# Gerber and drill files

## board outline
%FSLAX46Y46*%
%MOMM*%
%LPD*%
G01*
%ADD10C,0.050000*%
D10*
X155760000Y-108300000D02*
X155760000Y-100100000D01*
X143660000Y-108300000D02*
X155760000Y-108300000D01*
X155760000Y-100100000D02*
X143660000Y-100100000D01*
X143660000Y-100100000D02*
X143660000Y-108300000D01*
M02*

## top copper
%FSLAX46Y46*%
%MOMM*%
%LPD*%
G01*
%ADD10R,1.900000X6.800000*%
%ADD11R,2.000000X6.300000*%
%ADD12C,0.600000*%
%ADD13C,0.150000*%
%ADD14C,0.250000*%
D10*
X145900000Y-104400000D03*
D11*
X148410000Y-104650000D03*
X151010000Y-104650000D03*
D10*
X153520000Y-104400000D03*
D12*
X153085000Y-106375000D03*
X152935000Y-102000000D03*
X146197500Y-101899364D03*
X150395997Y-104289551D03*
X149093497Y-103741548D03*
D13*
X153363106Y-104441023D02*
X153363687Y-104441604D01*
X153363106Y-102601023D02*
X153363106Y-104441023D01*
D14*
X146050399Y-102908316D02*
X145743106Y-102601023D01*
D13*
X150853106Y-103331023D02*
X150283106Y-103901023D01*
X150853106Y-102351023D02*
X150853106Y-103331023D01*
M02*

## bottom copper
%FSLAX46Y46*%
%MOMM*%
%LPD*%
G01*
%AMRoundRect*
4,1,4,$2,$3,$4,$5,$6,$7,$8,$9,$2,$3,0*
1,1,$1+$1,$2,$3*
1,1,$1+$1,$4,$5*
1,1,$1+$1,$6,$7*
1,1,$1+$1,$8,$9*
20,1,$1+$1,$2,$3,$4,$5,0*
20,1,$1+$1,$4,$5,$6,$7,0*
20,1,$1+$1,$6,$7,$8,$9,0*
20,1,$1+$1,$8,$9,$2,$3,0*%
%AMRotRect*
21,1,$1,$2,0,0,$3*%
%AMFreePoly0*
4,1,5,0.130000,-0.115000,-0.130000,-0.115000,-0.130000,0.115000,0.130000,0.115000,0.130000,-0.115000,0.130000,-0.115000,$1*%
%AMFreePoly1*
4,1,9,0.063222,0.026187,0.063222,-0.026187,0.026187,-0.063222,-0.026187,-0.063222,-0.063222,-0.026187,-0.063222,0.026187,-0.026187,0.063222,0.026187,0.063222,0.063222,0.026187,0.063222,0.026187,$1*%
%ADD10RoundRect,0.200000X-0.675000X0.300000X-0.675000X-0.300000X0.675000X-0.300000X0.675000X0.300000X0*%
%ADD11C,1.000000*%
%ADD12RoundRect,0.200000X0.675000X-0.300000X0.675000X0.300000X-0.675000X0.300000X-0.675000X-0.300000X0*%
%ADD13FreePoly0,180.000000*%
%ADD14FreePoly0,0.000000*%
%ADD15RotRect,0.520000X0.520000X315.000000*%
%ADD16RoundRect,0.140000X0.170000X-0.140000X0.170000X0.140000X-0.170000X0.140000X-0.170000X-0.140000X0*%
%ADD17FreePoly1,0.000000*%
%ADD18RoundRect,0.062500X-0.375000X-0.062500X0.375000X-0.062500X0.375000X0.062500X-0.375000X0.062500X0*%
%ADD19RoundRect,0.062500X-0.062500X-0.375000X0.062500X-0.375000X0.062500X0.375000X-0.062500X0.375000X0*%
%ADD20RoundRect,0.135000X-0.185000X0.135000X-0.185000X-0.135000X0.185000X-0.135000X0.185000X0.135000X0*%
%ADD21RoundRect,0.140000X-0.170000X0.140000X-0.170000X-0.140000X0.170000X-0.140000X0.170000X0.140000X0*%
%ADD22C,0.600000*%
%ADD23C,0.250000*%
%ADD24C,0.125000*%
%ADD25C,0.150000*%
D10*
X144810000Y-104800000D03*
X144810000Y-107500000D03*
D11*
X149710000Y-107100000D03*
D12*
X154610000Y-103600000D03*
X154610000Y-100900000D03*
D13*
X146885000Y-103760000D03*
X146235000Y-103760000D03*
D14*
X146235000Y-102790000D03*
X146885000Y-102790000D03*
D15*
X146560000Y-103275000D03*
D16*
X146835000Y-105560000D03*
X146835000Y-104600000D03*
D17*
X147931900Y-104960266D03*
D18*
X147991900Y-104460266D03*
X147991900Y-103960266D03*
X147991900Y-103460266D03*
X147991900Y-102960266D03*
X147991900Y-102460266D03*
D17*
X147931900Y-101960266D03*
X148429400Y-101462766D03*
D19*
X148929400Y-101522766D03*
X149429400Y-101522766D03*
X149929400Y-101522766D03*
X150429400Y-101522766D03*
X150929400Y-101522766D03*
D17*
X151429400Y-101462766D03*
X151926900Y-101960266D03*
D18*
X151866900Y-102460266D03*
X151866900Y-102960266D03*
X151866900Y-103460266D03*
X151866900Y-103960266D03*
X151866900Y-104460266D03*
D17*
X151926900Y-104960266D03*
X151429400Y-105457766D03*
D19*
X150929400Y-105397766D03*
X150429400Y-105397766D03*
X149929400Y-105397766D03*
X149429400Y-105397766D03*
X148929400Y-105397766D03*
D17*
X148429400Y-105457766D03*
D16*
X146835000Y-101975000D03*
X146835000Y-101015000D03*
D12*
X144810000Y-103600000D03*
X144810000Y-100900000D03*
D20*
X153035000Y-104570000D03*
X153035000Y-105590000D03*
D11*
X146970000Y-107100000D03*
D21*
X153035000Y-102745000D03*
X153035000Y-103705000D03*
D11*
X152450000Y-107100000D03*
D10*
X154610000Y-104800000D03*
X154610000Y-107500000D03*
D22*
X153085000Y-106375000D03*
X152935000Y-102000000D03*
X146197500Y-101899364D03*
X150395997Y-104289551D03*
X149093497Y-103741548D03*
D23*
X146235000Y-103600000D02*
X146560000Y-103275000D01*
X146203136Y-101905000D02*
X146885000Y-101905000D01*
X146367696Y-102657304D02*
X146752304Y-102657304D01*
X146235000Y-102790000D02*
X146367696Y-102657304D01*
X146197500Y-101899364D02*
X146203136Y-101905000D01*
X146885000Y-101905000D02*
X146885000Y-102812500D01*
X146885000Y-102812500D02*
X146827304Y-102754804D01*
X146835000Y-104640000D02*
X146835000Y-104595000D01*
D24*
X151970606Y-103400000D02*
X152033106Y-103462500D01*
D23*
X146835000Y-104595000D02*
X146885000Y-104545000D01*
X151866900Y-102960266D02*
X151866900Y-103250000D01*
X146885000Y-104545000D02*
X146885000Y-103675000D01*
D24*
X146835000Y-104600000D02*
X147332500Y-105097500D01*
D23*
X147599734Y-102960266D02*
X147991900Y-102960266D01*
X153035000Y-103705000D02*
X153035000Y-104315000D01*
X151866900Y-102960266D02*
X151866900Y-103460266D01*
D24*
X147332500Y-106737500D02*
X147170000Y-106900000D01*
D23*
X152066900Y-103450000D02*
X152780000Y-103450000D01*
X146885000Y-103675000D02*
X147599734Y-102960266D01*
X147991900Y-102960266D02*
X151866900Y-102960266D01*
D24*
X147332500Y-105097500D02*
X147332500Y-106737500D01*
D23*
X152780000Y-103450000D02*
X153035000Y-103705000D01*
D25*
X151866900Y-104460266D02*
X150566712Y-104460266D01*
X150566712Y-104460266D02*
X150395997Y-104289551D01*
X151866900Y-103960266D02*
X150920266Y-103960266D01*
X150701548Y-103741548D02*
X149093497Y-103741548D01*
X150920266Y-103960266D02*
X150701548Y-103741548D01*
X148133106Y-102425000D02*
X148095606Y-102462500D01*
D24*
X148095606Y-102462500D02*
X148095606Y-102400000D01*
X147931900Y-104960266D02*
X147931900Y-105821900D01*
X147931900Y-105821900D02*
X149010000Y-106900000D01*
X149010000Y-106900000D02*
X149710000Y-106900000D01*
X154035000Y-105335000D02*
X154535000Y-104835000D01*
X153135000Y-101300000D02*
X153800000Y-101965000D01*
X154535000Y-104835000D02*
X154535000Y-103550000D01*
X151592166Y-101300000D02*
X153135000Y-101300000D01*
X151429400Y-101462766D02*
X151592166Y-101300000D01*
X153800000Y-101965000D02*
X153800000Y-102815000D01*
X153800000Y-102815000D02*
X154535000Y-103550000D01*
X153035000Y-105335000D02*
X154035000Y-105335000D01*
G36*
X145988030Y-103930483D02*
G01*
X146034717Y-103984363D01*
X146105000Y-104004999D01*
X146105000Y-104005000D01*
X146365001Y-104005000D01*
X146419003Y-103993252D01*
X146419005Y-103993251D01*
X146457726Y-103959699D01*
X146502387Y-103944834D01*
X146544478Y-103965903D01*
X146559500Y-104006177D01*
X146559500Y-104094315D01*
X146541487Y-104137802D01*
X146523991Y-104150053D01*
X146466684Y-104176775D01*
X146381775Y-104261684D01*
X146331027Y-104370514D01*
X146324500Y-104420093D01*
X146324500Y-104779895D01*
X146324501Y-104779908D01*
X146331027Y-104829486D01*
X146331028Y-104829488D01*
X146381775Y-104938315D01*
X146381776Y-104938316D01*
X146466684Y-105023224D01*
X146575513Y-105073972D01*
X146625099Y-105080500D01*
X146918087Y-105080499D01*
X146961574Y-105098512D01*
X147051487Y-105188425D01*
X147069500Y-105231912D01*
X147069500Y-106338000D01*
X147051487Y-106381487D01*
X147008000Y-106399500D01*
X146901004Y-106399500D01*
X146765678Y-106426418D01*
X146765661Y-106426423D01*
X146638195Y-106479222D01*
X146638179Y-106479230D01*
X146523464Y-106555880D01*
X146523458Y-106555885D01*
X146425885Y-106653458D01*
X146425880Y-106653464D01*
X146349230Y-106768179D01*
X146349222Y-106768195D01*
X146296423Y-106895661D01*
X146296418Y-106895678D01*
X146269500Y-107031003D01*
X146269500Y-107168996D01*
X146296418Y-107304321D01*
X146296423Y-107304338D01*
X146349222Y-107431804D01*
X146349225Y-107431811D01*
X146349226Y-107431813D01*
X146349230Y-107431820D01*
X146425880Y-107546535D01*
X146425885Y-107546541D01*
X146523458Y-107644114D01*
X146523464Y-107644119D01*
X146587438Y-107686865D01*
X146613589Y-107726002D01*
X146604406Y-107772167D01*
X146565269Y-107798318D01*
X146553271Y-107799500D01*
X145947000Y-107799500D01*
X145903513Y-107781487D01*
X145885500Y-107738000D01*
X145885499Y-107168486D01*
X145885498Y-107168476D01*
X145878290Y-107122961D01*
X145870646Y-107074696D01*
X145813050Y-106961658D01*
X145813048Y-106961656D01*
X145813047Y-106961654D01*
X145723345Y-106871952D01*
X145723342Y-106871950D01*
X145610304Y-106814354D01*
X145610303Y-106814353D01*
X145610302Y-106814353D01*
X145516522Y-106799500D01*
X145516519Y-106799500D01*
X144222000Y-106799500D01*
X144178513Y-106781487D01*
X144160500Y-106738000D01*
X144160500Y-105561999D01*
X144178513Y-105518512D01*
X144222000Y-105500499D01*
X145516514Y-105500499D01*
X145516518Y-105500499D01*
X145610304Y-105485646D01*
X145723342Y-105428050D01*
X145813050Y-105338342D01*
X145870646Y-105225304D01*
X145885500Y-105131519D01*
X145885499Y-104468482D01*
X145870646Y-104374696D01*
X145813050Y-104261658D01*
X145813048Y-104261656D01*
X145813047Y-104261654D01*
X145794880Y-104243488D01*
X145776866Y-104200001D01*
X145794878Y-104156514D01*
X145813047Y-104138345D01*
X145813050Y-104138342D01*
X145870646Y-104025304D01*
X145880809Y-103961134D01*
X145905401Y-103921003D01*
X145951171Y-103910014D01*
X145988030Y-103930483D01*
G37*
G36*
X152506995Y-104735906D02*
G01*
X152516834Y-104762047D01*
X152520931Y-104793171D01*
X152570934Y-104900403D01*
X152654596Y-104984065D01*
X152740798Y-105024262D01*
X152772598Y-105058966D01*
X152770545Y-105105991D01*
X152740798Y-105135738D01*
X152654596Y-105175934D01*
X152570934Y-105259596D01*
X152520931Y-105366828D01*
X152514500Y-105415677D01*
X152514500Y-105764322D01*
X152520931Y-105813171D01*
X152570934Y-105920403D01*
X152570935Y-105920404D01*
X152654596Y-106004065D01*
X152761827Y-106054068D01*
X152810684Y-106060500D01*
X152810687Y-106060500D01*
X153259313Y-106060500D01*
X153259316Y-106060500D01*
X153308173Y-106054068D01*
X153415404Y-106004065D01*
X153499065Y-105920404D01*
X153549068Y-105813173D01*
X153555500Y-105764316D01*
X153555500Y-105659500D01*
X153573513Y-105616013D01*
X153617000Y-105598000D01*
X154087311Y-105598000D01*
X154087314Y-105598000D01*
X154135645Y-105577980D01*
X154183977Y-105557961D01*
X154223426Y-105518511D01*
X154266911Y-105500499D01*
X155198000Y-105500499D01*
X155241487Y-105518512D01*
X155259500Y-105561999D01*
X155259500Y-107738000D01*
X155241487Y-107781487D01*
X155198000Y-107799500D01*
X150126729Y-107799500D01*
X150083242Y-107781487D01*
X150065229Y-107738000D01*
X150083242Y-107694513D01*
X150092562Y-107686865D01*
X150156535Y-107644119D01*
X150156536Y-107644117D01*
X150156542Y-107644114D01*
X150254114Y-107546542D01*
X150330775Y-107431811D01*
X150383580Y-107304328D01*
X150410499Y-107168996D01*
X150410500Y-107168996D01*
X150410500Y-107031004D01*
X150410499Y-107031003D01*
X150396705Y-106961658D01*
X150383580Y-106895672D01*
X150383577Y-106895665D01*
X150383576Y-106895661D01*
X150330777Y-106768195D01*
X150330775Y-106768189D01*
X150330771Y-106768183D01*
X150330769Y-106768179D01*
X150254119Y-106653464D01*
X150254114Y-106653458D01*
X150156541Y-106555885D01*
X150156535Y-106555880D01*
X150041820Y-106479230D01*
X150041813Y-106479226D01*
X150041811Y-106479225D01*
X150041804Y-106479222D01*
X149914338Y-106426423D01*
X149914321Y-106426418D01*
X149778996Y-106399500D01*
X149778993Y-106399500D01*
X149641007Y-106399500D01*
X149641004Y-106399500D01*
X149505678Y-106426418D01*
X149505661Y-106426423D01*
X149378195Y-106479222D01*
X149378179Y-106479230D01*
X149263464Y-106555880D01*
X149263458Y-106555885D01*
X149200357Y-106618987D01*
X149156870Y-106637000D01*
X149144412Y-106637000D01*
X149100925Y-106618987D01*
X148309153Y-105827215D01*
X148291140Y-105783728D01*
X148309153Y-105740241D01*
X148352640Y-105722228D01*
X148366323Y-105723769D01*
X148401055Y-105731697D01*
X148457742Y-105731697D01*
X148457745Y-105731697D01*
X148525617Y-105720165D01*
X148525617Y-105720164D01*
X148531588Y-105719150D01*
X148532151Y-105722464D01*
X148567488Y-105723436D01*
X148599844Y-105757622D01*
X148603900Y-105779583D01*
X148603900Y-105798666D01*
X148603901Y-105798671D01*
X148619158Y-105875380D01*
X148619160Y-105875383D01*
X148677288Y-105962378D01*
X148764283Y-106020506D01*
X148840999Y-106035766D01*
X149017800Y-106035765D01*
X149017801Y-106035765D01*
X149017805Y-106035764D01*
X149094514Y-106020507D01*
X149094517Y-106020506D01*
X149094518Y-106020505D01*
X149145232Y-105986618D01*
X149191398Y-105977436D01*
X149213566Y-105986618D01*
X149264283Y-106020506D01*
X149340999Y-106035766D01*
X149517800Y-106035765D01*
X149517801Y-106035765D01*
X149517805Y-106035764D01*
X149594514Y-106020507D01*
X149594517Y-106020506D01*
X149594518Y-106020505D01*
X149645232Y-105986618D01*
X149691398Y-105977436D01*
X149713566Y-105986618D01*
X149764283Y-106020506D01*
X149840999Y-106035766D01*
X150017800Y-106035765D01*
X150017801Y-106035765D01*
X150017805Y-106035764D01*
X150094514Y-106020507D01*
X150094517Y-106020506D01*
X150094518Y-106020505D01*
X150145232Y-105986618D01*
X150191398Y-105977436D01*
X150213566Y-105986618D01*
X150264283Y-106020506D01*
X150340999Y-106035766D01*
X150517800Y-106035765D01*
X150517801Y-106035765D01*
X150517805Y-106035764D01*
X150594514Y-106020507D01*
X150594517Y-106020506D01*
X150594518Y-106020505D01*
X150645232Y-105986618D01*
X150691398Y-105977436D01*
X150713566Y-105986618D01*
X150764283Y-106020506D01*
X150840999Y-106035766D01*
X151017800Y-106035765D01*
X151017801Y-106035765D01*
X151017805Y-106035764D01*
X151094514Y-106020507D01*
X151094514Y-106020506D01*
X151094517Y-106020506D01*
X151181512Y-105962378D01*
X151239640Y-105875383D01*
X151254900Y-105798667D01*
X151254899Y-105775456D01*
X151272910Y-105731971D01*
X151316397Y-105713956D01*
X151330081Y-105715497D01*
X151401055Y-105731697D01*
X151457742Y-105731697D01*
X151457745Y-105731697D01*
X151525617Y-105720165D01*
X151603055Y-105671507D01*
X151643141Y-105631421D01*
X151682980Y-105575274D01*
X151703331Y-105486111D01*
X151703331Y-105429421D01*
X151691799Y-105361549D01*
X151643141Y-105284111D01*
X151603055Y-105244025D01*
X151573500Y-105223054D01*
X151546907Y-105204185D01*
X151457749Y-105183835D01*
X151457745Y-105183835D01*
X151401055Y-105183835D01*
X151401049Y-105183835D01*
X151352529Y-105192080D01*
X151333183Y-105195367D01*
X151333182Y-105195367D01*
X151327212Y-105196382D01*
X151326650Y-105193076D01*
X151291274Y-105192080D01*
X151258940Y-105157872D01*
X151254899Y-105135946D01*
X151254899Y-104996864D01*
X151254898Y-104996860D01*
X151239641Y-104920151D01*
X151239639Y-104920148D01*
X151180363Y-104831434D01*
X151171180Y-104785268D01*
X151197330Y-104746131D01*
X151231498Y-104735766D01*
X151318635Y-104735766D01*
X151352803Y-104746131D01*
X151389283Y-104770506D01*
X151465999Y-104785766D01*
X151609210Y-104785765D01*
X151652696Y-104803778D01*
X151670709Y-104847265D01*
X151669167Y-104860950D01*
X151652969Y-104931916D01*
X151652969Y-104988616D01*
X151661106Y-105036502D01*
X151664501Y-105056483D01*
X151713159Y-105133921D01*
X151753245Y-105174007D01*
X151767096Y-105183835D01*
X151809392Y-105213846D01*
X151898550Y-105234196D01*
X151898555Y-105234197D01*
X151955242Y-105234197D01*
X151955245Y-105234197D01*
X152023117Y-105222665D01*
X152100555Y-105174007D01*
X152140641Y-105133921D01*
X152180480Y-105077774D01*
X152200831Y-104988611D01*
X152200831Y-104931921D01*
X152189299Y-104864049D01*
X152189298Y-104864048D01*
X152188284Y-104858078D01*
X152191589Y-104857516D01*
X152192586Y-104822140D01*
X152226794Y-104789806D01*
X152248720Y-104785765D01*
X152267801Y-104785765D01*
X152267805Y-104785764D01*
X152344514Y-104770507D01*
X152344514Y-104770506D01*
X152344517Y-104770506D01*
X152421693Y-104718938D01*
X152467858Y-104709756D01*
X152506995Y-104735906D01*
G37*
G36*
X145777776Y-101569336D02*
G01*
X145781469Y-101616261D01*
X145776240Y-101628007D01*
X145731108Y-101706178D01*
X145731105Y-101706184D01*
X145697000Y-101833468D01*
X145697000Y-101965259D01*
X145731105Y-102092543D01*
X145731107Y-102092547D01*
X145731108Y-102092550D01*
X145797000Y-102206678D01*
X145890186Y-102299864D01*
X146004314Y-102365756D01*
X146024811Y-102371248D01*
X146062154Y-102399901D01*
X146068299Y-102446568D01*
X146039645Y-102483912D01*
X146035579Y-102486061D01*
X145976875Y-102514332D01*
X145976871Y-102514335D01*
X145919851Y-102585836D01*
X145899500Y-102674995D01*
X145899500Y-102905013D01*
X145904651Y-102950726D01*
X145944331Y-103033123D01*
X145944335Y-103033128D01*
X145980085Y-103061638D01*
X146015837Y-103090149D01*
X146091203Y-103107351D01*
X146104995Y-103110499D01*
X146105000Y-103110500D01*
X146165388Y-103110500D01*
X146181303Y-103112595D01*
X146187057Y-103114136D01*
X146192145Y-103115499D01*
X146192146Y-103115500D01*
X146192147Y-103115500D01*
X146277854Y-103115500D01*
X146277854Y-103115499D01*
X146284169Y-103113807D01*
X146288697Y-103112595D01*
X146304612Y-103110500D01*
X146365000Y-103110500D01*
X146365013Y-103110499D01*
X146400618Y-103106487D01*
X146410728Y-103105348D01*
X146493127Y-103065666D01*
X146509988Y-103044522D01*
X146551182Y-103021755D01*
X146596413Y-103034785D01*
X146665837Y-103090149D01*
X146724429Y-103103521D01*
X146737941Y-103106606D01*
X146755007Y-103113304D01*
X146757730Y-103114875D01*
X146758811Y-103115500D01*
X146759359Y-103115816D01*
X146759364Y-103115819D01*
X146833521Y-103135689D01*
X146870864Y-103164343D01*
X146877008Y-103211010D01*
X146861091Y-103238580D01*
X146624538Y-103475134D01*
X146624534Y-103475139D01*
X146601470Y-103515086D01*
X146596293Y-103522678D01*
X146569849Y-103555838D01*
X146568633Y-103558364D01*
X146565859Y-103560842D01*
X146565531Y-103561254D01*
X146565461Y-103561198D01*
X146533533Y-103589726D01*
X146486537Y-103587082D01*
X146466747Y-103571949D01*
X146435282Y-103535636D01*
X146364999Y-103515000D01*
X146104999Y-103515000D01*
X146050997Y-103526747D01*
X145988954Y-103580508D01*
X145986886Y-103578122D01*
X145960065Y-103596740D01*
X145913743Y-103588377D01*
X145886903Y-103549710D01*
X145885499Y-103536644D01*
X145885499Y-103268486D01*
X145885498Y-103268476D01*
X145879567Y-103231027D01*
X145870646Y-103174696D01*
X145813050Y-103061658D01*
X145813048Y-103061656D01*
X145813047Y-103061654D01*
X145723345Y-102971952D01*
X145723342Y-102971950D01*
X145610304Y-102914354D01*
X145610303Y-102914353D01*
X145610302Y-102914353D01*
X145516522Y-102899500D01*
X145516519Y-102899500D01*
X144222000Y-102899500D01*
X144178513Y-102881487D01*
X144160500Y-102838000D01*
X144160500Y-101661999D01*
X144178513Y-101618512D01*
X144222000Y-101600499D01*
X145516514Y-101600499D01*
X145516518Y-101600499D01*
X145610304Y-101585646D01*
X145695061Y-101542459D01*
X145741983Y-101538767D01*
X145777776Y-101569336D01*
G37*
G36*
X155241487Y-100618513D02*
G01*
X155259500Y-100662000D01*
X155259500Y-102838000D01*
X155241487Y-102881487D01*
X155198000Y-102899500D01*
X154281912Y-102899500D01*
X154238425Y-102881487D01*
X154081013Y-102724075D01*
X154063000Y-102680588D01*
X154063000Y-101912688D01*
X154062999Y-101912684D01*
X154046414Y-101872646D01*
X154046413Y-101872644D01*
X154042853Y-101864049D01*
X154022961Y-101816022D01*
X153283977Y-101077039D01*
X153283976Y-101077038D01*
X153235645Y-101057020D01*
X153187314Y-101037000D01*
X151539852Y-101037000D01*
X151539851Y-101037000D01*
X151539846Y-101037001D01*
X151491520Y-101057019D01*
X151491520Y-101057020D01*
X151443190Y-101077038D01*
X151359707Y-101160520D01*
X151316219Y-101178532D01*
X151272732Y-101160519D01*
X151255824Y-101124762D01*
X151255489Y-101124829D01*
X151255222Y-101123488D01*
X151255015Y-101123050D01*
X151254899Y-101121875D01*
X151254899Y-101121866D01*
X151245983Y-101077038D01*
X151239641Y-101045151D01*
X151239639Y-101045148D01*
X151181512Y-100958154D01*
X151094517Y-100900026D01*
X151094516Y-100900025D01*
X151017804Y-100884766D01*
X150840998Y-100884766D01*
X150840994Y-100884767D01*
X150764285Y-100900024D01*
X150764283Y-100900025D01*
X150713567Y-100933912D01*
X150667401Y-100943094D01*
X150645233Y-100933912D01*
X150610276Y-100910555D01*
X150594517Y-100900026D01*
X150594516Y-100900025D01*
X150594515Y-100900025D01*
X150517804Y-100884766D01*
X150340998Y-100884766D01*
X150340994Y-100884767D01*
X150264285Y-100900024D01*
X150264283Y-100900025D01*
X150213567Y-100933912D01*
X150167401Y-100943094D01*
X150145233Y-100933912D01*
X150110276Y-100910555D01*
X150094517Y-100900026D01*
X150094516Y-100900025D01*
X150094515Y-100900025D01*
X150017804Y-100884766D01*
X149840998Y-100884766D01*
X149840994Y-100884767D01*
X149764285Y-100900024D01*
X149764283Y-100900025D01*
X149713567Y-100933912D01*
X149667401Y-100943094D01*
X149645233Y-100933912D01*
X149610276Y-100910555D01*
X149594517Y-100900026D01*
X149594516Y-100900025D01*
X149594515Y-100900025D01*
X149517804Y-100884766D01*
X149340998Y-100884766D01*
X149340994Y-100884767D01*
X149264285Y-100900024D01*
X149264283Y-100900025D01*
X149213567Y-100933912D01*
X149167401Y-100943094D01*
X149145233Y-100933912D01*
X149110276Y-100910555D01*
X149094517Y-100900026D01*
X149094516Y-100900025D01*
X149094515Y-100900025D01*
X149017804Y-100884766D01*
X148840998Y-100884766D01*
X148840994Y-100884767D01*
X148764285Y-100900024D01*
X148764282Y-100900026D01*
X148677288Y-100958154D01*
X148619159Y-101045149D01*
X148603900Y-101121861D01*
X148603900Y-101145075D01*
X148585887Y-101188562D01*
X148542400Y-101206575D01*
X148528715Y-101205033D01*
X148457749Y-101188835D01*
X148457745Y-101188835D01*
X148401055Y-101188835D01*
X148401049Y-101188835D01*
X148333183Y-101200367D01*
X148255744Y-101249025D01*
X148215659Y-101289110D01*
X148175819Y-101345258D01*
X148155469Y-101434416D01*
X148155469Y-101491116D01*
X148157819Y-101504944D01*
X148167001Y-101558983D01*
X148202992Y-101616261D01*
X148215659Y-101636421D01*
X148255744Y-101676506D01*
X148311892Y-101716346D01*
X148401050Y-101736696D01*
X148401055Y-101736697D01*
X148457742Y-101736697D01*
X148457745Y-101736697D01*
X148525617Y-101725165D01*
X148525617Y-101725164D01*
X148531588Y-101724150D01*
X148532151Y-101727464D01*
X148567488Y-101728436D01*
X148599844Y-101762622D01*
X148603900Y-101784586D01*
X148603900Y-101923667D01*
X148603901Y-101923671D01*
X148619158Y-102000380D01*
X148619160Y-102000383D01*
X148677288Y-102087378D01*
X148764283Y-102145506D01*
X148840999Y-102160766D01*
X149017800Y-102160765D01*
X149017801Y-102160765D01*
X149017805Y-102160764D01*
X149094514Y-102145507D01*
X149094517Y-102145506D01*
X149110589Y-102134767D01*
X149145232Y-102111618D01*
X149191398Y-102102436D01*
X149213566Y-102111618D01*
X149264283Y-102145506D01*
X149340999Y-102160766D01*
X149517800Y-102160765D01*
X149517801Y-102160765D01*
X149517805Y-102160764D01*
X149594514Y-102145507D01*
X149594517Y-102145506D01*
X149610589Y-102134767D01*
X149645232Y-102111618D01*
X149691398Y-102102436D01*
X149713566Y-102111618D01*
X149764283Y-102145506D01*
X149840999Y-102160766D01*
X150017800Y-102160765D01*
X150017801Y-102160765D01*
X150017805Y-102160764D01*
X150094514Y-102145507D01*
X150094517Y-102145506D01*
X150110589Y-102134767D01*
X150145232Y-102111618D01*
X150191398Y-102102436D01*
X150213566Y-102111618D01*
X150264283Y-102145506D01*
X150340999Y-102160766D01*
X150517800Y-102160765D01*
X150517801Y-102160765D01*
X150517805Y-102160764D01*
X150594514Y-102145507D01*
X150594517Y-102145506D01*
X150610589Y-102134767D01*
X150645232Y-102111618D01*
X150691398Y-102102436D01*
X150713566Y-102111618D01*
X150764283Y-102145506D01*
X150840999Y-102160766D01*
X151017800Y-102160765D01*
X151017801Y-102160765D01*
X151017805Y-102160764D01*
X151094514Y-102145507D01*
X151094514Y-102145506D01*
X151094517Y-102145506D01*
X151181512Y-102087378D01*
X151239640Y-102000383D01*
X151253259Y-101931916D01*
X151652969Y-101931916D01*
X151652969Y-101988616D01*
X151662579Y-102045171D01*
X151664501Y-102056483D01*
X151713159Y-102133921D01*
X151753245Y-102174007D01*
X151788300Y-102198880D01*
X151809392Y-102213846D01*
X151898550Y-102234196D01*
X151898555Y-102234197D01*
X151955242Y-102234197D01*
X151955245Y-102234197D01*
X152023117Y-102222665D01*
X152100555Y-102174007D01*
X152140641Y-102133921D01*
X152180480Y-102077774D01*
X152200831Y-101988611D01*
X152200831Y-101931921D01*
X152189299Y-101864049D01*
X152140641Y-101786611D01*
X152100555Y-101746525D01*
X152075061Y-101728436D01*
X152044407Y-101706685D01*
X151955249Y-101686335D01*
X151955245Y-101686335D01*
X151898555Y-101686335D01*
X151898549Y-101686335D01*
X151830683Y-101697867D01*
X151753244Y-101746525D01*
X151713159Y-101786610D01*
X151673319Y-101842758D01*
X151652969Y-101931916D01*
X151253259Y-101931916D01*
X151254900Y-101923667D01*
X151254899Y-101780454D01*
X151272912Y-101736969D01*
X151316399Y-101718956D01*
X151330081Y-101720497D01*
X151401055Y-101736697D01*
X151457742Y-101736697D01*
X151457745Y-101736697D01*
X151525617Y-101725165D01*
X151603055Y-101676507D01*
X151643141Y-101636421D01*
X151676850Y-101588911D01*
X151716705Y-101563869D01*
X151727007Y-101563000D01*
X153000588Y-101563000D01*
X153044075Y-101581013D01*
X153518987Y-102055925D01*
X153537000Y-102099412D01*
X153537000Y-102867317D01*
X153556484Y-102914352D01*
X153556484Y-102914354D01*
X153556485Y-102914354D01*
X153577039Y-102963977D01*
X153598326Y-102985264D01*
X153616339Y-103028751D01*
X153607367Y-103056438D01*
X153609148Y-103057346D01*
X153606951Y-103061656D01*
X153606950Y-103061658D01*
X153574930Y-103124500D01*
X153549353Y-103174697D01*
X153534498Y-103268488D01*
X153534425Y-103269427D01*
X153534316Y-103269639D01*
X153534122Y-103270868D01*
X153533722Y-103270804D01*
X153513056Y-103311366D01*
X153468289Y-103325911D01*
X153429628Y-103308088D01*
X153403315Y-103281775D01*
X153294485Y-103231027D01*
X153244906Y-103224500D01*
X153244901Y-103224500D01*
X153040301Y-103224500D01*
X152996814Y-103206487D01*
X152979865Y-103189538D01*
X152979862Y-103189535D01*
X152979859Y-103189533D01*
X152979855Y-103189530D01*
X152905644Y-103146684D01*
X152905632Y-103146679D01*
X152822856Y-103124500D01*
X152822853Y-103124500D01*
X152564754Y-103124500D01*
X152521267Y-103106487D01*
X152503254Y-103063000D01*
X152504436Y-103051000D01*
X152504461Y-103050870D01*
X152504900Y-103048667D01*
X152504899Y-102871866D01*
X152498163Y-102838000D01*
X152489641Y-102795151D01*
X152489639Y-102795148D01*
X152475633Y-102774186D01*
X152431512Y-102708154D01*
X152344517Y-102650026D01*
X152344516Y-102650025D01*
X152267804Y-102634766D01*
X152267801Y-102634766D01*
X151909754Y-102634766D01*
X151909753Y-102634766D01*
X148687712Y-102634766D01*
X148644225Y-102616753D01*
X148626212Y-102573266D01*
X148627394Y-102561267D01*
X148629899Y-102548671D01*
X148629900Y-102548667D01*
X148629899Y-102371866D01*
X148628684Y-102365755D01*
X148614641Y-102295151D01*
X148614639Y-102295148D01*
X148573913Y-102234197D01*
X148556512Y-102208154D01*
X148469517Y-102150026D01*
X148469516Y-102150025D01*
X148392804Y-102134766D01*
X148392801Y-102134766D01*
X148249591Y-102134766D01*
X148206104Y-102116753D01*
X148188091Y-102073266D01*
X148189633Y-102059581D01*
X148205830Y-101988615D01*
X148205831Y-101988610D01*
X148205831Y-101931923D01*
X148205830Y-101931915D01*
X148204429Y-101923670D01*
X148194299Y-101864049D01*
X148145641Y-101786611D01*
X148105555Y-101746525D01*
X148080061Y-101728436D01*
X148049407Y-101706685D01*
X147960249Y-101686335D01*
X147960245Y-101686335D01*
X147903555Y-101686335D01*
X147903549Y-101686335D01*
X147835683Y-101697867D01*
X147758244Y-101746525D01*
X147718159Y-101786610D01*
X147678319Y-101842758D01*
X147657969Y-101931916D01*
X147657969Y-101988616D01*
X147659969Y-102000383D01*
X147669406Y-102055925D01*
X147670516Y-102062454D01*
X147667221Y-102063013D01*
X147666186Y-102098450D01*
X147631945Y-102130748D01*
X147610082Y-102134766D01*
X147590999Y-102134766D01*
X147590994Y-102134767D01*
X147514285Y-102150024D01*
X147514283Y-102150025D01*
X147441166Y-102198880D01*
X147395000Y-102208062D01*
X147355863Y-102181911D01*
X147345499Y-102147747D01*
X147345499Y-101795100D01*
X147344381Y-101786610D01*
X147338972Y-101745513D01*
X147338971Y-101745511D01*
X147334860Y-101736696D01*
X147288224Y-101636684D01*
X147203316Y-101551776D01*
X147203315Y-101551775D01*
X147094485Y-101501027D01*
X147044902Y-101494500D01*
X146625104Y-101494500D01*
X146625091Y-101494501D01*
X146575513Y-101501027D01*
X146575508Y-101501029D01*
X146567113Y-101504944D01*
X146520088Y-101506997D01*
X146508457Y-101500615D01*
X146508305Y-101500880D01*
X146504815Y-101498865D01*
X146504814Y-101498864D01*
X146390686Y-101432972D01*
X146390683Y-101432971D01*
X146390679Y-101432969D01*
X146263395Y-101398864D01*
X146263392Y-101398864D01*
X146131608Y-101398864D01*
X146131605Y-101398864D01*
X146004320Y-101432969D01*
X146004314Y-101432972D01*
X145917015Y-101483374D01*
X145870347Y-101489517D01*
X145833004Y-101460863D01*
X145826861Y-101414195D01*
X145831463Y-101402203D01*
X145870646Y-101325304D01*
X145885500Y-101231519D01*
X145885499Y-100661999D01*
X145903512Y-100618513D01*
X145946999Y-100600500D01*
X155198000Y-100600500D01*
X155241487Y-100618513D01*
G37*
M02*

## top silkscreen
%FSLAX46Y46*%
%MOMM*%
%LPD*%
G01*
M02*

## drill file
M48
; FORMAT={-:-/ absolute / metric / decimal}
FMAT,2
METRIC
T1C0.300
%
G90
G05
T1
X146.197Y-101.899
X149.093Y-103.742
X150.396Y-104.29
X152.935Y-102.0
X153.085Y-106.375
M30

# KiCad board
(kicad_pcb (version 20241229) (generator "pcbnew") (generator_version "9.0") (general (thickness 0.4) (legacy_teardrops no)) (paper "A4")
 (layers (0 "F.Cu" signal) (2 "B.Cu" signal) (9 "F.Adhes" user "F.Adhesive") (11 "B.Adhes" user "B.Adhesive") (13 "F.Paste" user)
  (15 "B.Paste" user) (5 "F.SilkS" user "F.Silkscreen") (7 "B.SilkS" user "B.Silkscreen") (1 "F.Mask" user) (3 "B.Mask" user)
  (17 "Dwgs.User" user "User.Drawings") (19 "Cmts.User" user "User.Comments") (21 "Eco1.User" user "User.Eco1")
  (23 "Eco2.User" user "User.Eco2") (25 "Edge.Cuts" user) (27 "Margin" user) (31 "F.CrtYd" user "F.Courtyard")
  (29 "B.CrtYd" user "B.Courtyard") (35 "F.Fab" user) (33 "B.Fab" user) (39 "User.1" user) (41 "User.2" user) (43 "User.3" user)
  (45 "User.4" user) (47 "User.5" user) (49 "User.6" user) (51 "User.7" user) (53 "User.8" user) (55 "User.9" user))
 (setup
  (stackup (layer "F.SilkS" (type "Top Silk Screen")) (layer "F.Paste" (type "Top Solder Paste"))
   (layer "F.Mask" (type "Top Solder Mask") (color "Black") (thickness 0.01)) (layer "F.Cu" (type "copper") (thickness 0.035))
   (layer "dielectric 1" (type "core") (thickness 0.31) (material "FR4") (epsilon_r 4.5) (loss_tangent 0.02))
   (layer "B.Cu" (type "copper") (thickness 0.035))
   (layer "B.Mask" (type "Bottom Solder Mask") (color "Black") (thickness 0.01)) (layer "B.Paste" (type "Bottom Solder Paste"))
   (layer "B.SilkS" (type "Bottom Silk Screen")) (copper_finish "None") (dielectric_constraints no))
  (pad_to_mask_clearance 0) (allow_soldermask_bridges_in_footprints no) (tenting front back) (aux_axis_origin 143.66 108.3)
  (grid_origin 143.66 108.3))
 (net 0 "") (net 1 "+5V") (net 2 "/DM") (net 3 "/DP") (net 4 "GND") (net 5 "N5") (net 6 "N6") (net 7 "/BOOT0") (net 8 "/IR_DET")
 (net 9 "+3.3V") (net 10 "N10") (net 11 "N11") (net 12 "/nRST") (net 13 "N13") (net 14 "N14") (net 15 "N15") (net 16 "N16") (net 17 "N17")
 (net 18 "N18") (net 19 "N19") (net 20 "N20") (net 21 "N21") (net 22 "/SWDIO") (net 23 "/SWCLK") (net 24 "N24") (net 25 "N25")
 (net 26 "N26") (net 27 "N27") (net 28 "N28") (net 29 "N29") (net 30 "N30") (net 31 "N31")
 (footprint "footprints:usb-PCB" (layer "F.Cu") (at 149.71 100.1 180)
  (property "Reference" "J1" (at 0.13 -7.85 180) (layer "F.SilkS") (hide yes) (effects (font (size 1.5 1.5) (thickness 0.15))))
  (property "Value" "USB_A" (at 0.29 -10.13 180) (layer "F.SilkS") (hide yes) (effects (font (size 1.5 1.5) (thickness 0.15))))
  (pad "1" connect rect (at 3.81 -4.3 180) (size 1.9 6.8) (layers "F.Cu" "F.Mask") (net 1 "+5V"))
  (pad "2" connect rect (at 1.3 -4.55 180) (size 2 6.3) (layers "F.Cu" "F.Mask") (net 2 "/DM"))
  (pad "3" connect rect (at -1.3 -4.55 180) (size 2 6.3) (layers "F.Cu" "F.Mask") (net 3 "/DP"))
  (pad "4" connect rect (at -3.81 -4.3 180) (size 1.9 6.8) (layers "F.Cu" "F.Mask") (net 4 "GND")))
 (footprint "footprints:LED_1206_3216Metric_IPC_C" (layer "B.Cu") (at 144.81 106.15 -90)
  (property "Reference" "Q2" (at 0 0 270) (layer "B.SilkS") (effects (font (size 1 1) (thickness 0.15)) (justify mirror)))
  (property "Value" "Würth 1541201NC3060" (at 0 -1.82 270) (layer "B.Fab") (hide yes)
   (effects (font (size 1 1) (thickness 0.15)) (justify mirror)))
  (pad "1" smd roundrect (at -1.35 0 270) (size 1 1.75) (layers "B.Cu" "B.Mask" "B.Paste") (roundrect_rratio 0.2) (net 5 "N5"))
  (pad "2" smd roundrect (at 1.35 0 270) (size 1 1.75) (layers "B.Cu" "B.Mask" "B.Paste") (roundrect_rratio 0.2) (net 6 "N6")))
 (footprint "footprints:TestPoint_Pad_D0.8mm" (layer "B.Cu") (at 150.01 106.55 180)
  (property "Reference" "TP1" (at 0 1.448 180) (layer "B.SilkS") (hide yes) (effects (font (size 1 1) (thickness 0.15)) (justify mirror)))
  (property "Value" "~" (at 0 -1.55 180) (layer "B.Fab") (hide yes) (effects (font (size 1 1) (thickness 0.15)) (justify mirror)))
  (pad "1" smd circle (at 0.3 -0.55 180) (size 1 1) (layers "B.Cu" "B.Mask") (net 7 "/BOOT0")))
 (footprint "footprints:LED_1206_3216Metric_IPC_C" (layer "B.Cu") (at 154.61 102.25 90)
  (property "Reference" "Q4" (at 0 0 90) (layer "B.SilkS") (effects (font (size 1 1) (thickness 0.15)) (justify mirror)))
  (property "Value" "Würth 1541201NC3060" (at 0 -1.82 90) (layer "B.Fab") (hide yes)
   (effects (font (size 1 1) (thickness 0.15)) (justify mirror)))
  (pad "1" smd roundrect (at -1.35 0 90) (size 1 1.75) (layers "B.Cu" "B.Mask" "B.Paste") (roundrect_rratio 0.2) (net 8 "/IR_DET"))
  (pad "2" smd roundrect (at 1.35 0 90) (size 1 1.75) (layers "B.Cu" "B.Mask" "B.Paste") (roundrect_rratio 0.2) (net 4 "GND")))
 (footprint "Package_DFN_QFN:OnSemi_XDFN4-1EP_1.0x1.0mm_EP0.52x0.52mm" (layer "B.Cu") (at 146.56 103.275 90)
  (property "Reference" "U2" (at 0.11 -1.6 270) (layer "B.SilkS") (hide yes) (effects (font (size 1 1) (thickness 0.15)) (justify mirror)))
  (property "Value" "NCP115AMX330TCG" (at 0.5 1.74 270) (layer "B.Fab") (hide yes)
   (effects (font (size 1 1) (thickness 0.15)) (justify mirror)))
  (pad "1" smd custom (at -0.485 0.325 180) (size 0.26 0.23) (layers "B.Cu" "B.Mask" "B.Paste") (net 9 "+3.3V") (zone_connect 0)
   (thermal_bridge_angle 45) (options (clearance outline) (anchor rect)) (primitives))
  (pad "2" smd custom (at -0.485 -0.325 180) (size 0.26 0.23) (layers "B.Cu" "B.Mask" "B.Paste") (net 4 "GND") (zone_connect 0)
   (thermal_bridge_angle 45) (options (clearance outline) (anchor rect)) (primitives))
  (pad "3" smd custom (at 0.485 -0.325) (size 0.26 0.23) (layers "B.Cu" "B.Mask" "B.Paste") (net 1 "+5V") (zone_connect 0)
   (thermal_bridge_angle 45) (options (clearance outline) (anchor rect)) (primitives))
  (pad "4" smd custom (at 0.485 0.325) (size 0.26 0.23) (layers "B.Cu" "B.Mask" "B.Paste") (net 1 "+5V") (zone_connect 0)
   (thermal_bridge_angle 45) (options (clearance outline) (anchor rect)) (primitives))
  (pad "5" smd rect (at 0 0 315) (size 0.52 0.52) (layers "B.Cu" "B.Mask" "B.Paste") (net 4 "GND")))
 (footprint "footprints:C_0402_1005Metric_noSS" (layer "B.Cu") (at 146.835 105.08 90)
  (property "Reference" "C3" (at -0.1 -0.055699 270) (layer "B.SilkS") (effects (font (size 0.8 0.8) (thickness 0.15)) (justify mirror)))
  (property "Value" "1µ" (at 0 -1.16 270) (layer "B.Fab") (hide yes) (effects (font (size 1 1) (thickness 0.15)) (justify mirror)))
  (pad "1" smd roundrect (at -0.48 0 90) (size 0.56 0.62) (layers "B.Cu" "B.Mask" "B.Paste") (roundrect_rratio 0.25) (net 4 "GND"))
  (pad "2" smd roundrect (at 0.48 0 90) (size 0.56 0.62) (layers "B.Cu" "B.Mask" "B.Paste") (roundrect_rratio 0.25) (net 9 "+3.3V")))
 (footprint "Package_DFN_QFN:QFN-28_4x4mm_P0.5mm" (layer "B.Cu") (at 149.9294 103.460266)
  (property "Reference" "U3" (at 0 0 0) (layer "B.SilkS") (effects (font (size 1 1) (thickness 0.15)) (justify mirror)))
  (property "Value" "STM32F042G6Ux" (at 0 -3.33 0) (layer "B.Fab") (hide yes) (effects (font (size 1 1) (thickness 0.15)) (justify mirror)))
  (pad "1" smd custom (at -1.9975 1.5) (size 0.136863 0.136863) (layers "B.Cu" "B.Mask" "B.Paste") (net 7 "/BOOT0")
   (options (clearance outline) (anchor circle)) (primitives))
  (pad "2" smd roundrect (at -1.9375 1) (size 0.875 0.25) (layers "B.Cu" "B.Mask" "B.Paste") (roundrect_rratio 0.25) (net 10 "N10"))
  (pad "3" smd roundrect (at -1.9375 0.5) (size 0.875 0.25) (layers "B.Cu" "B.Mask" "B.Paste") (roundrect_rratio 0.25) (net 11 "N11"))
  (pad "4" smd roundrect (at -1.9375 0) (size 0.875 0.25) (layers "B.Cu" "B.Mask" "B.Paste") (roundrect_rratio 0.25) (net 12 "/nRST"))
  (pad "5" smd roundrect (at -1.9375 -0.5) (size 0.875 0.25) (layers "B.Cu" "B.Mask" "B.Paste") (roundrect_rratio 0.25) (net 9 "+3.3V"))
  (pad "6" smd roundrect (at -1.9375 -1) (size 0.875 0.25) (layers "B.Cu" "B.Mask" "B.Paste") (roundrect_rratio 0.25) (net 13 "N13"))
  (pad "7" smd custom (at -1.9975 -1.5) (size 0.136863 0.136863) (layers "B.Cu" "B.Mask" "B.Paste") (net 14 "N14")
   (options (clearance outline) (anchor circle)) (primitives))
  (pad "8" smd custom (at -1.5 -1.9975) (size 0.136863 0.136863) (layers "B.Cu" "B.Mask" "B.Paste") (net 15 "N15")
   (options (clearance outline) (anchor circle)) (primitives))
  (pad "9" smd roundrect (at -1 -1.9375) (size 0.25 0.875) (layers "B.Cu" "B.Mask" "B.Paste") (roundrect_rratio 0.25) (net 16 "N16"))
  (pad "10" smd roundrect (at -0.5 -1.9375) (size 0.25 0.875) (layers "B.Cu" "B.Mask" "B.Paste") (roundrect_rratio 0.25) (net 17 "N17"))
  (pad "11" smd roundrect (at 0 -1.9375) (size 0.25 0.875) (layers "B.Cu" "B.Mask" "B.Paste") (roundrect_rratio 0.25) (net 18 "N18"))
  (pad "12" smd roundrect (at 0.5 -1.9375) (size 0.25 0.875) (layers "B.Cu" "B.Mask" "B.Paste") (roundrect_rratio 0.25) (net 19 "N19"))
  (pad "13" smd roundrect (at 1 -1.9375) (size 0.25 0.875) (layers "B.Cu" "B.Mask" "B.Paste") (roundrect_rratio 0.25) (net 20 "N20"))
  (pad "14" smd custom (at 1.5 -1.9975) (size 0.136863 0.136863) (layers "B.Cu" "B.Mask" "B.Paste") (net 8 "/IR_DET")
   (options (clearance outline) (anchor circle)) (primitives))
  (pad "15" smd custom (at 1.9975 -1.5) (size 0.136863 0.136863) (layers "B.Cu" "B.Mask" "B.Paste") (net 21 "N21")
   (options (clearance outline) (anchor circle)) (primitives))
  (pad "16" smd roundrect (at 1.9375 -1) (size 0.875 0.25) (layers "B.Cu" "B.Mask" "B.Paste") (roundrect_rratio 0.25) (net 4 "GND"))
  (pad "17" smd roundrect (at 1.9375 -0.5) (size 0.875 0.25) (layers "B.Cu" "B.Mask" "B.Paste") (roundrect_rratio 0.25) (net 9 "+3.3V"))
  (pad "18" smd roundrect (at 1.9375 0) (size 0.875 0.25) (layers "B.Cu" "B.Mask" "B.Paste") (roundrect_rratio 0.25) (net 9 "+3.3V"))
  (pad "19" smd roundrect (at 1.9375 0.5) (size 0.875 0.25) (layers "B.Cu" "B.Mask" "B.Paste") (roundrect_rratio 0.25) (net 2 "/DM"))
  (pad "20" smd roundrect (at 1.9375 1) (size 0.875 0.25) (layers "B.Cu" "B.Mask" "B.Paste") (roundrect_rratio 0.25) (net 3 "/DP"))
  (pad "21" smd custom (at 1.9975 1.5) (size 0.136863 0.136863) (layers "B.Cu" "B.Mask" "B.Paste") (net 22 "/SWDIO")
   (options (clearance outline) (anchor circle)) (primitives))
  (pad "22" smd custom (at 1.5 1.9975) (size 0.136863 0.136863) (layers "B.Cu" "B.Mask" "B.Paste") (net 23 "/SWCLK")
   (options (clearance outline) (anchor circle)) (primitives))
  (pad "23" smd roundrect (at 1 1.9375) (size 0.25 0.875) (layers "B.Cu" "B.Mask" "B.Paste") (roundrect_rratio 0.25) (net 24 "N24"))
  (pad "24" smd roundrect (at 0.5 1.9375) (size 0.25 0.875) (layers "B.Cu" "B.Mask" "B.Paste") (roundrect_rratio 0.25) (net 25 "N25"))
  (pad "25" smd roundrect (at 0 1.9375) (size 0.25 0.875) (layers "B.Cu" "B.Mask" "B.Paste") (roundrect_rratio 0.25) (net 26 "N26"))
  (pad "26" smd roundrect (at -0.5 1.9375) (size 0.25 0.875) (layers "B.Cu" "B.Mask" "B.Paste") (roundrect_rratio 0.25) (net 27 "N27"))
  (pad "27" smd roundrect (at -1 1.9375) (size 0.25 0.875) (layers "B.Cu" "B.Mask" "B.Paste") (roundrect_rratio 0.25) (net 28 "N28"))
  (pad "28" smd custom (at -1.5 1.9975) (size 0.136863 0.136863) (layers "B.Cu" "B.Mask" "B.Paste") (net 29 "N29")
   (options (clearance outline) (anchor circle)) (primitives)))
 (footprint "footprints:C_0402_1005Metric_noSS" (layer "B.Cu") (at 146.835 101.495 90)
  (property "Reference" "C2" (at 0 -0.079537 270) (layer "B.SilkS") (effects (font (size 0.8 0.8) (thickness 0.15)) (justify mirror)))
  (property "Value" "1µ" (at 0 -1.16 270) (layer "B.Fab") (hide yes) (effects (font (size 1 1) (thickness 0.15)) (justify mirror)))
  (pad "1" smd roundrect (at -0.48 0 90) (size 0.56 0.62) (layers "B.Cu" "B.Mask" "B.Paste") (roundrect_rratio 0.25) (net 1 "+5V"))
  (pad "2" smd roundrect (at 0.48 0 90) (size 0.56 0.62) (layers "B.Cu" "B.Mask" "B.Paste") (roundrect_rratio 0.25) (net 4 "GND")))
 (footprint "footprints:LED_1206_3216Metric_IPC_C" (layer "B.Cu") (at 144.81 102.25 90)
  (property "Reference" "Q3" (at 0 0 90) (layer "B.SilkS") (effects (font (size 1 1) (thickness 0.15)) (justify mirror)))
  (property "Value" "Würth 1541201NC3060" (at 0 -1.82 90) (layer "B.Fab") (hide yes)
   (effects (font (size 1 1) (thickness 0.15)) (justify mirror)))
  (pad "1" smd roundrect (at -1.35 0 90) (size 1 1.75) (layers "B.Cu" "B.Mask" "B.Paste") (roundrect_rratio 0.2) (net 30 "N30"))
  (pad "2" smd roundrect (at 1.35 0 90) (size 1 1.75) (layers "B.Cu" "B.Mask" "B.Paste") (roundrect_rratio 0.2) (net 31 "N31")))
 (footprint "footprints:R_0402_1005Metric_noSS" (layer "B.Cu") (at 153.035 105.08 -90)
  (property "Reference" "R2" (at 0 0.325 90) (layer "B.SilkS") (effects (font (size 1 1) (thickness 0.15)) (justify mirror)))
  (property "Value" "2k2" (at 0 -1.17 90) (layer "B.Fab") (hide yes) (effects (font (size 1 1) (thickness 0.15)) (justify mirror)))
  (pad "1" smd roundrect (at -0.51 0 270) (size 0.54 0.64) (layers "B.Cu" "B.Mask" "B.Paste") (roundrect_rratio 0.25) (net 9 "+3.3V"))
  (pad "2" smd roundrect (at 0.51 0 270) (size 0.54 0.64) (layers "B.Cu" "B.Mask" "B.Paste") (roundrect_rratio 0.25) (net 8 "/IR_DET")))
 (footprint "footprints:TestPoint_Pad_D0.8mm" (layer "B.Cu") (at 148.41 106.55)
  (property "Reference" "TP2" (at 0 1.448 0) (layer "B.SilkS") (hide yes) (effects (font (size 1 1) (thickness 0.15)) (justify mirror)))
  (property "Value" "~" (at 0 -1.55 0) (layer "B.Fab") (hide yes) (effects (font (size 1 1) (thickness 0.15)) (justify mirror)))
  (pad "1" smd circle (at -1.44 0.55) (size 1 0.8) (layers "B.Cu" "B.Mask") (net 9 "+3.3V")))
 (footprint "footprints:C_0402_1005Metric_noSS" (layer "B.Cu") (at 153.035 103.225 -90)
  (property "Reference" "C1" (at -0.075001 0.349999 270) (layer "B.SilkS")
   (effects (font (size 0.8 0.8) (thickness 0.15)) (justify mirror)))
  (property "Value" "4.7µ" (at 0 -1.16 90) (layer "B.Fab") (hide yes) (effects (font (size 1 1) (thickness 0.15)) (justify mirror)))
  (pad "1" smd roundrect (at -0.48 0 270) (size 0.56 0.62) (layers "B.Cu" "B.Mask" "B.Paste") (roundrect_rratio 0.25) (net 4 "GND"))
  (pad "2" smd roundrect (at 0.48 0 270) (size 0.56 0.62) (layers "B.Cu" "B.Mask" "B.Paste") (roundrect_rratio 0.25) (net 9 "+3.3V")))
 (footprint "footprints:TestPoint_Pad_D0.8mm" (layer "B.Cu") (at 159.385 106.9 180)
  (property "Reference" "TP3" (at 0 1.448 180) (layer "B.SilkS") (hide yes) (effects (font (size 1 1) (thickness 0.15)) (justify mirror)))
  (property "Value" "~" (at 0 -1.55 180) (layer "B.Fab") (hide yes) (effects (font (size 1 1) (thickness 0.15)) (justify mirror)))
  (pad "1" smd circle (at 6.935 -0.2 180) (size 1 0.8) (layers "B.Cu" "B.Mask") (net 4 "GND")))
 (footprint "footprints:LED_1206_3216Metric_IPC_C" (layer "B.Cu") (at 154.61 106.15 -90)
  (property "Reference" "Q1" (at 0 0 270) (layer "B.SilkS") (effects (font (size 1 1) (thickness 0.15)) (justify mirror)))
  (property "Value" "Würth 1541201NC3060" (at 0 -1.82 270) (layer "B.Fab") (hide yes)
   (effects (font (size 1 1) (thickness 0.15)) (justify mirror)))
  (pad "1" smd roundrect (at -1.35 0 270) (size 1 1.75) (layers "B.Cu" "B.Mask" "B.Paste") (roundrect_rratio 0.2) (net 8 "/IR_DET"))
  (pad "2" smd roundrect (at 1.35 0 270) (size 1 1.75) (layers "B.Cu" "B.Mask" "B.Paste") (roundrect_rratio 0.2) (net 4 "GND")))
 (gr_line (start 155.76 108.3) (end 155.76 100.1) (stroke (width 0.05) (type default)) (layer "Edge.Cuts"))
 (gr_line (start 143.66 108.3) (end 155.76 108.3) (stroke (width 0.05) (type default)) (layer "Edge.Cuts"))
 (gr_line (start 155.76 100.1) (end 143.66 100.1) (stroke (width 0.05) (type default)) (layer "Edge.Cuts"))
 (gr_line (start 143.66 100.1) (end 143.66 108.3) (stroke (width 0.05) (type default)) (layer "Edge.Cuts"))
 (segment (start 153.363106 104.441023) (end 153.363687 104.441604) (width 0.15) (layer "F.Cu") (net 4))
 (segment (start 153.363106 102.601023) (end 153.363106 104.441023) (width 0.15) (layer "F.Cu") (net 4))
 (via (at 153.085 106.375) (size 0.6) (drill 0.3) (layers "F.Cu" "B.Cu") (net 4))
 (via (at 152.935 102) (size 0.6) (drill 0.3) (layers "F.Cu" "B.Cu") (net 4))
 (segment (start 146.235 103.6) (end 146.56 103.275) (width 0.25) (layer "B.Cu") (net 4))
 (segment (start 146.050399 102.908316) (end 145.743106 102.601023) (width 0.25) (layer "F.Cu") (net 1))
 (via (at 146.1975 101.899364) (size 0.6) (drill 0.3) (layers "F.Cu" "B.Cu") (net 1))
 (segment (start 146.203136 101.905) (end 146.885 101.905) (width 0.25) (layer "B.Cu") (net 1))
 (segment (start 146.367696 102.657304) (end 146.752304 102.657304) (width 0.25) (layer "B.Cu") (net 1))
 (segment (start 146.235 102.79) (end 146.367696 102.657304) (width 0.25) (layer "B.Cu") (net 1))
 (segment (start 146.1975 101.899364) (end 146.203136 101.905) (width 0.25) (layer "B.Cu") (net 1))
 (segment (start 146.885 101.905) (end 146.885 102.8125) (width 0.25) (layer "B.Cu") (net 1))
 (segment (start 146.885 102.8125) (end 146.827304 102.754804) (width 0.25) (layer "B.Cu") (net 1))
 (segment (start 146.835 104.64) (end 146.835 104.595) (width 0.25) (layer "B.Cu") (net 9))
 (segment (start 151.970606 103.4) (end 152.033106 103.4625) (width 0.125) (layer "B.Cu") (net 9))
 (segment (start 146.835 104.595) (end 146.885 104.545) (width 0.25) (layer "B.Cu") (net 9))
 (segment (start 151.8669 102.960266) (end 151.8669 103.25) (width 0.25) (layer "B.Cu") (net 9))
 (segment (start 146.885 104.545) (end 146.885 103.675) (width 0.25) (layer "B.Cu") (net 9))
 (segment (start 146.835 104.6) (end 147.3325 105.0975) (width 0.125) (layer "B.Cu") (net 9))
 (segment (start 147.599734 102.960266) (end 147.9919 102.960266) (width 0.25) (layer "B.Cu") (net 9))
 (segment (start 153.035 103.705) (end 153.035 104.315) (width 0.25) (layer "B.Cu") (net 9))
 (segment (start 151.8669 102.960266) (end 151.8669 103.460266) (width 0.25) (layer "B.Cu") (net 9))
 (segment (start 147.3325 106.7375) (end 147.17 106.9) (width 0.125) (layer "B.Cu") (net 9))
 (segment (start 152.0669 103.45) (end 152.78 103.45) (width 0.25) (layer "B.Cu") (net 9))
 (segment (start 146.885 103.675) (end 147.599734 102.960266) (width 0.25) (layer "B.Cu") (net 9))
 (segment (start 147.9919 102.960266) (end 151.8669 102.960266) (width 0.25) (layer "B.Cu") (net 9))
 (segment (start 147.3325 105.0975) (end 147.3325 106.7375) (width 0.125) (layer "B.Cu") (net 9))
 (segment (start 152.78 103.45) (end 153.035 103.705) (width 0.25) (layer "B.Cu") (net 9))
 (segment (start 150.853106 103.331023) (end 150.283106 103.901023) (width 0.15) (layer "F.Cu") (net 3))
 (segment (start 150.853106 102.351023) (end 150.853106 103.331023) (width 0.15) (layer "F.Cu") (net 3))
 (via (at 150.395997 104.289551) (size 0.6) (drill 0.3) (layers "F.Cu" "B.Cu") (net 3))
 (segment (start 151.8669 104.460266) (end 150.566712 104.460266) (width 0.15) (layer "B.Cu") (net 3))
 (segment (start 150.566712 104.460266) (end 150.395997 104.289551) (width 0.15) (layer "B.Cu") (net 3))
 (via (at 149.093497 103.741548) (size 0.6) (drill 0.3) (layers "F.Cu" "B.Cu") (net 2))
 (segment (start 151.8669 103.960266) (end 150.920266 103.960266) (width 0.15) (layer "B.Cu") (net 2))
 (segment (start 150.701548 103.741548) (end 149.093497 103.741548) (width 0.15) (layer "B.Cu") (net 2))
 (segment (start 150.920266 103.960266) (end 150.701548 103.741548) (width 0.15) (layer "B.Cu") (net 2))
 (segment (start 148.133106 102.425) (end 148.095606 102.4625) (width 0.15) (layer "B.Cu") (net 13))
 (segment (start 148.095606 102.4625) (end 148.095606 102.4) (width 0.125) (layer "B.Cu") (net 13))
 (segment (start 147.9319 104.960266) (end 147.9319 105.8219) (width 0.125) (layer "B.Cu") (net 7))
 (segment (start 147.9319 105.8219) (end 149.01 106.9) (width 0.125) (layer "B.Cu") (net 7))
 (segment (start 149.01 106.9) (end 149.71 106.9) (width 0.125) (layer "B.Cu") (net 7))
 (segment (start 154.035 105.335) (end 154.535 104.835) (width 0.125) (layer "B.Cu") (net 8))
 (segment (start 153.135 101.3) (end 153.8 101.965) (width 0.125) (layer "B.Cu") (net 8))
 (segment (start 154.535 104.835) (end 154.535 103.55) (width 0.125) (layer "B.Cu") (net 8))
 (segment (start 151.592166 101.3) (end 153.135 101.3) (width 0.125) (layer "B.Cu") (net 8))
 (segment (start 151.4294 101.462766) (end 151.592166 101.3) (width 0.125) (layer "B.Cu") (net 8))
 (segment (start 153.8 101.965) (end 153.8 102.815) (width 0.125) (layer "B.Cu") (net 8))
 (segment (start 153.8 102.815) (end 154.535 103.55) (width 0.125) (layer "B.Cu") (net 8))
 (segment (start 153.035 105.335) (end 154.035 105.335) (width 0.125) (layer "B.Cu") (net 8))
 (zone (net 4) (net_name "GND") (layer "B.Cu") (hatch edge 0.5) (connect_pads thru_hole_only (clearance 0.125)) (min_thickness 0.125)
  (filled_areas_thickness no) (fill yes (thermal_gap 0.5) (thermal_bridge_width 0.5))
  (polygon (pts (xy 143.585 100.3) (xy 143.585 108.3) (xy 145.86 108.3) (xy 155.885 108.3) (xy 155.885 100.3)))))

